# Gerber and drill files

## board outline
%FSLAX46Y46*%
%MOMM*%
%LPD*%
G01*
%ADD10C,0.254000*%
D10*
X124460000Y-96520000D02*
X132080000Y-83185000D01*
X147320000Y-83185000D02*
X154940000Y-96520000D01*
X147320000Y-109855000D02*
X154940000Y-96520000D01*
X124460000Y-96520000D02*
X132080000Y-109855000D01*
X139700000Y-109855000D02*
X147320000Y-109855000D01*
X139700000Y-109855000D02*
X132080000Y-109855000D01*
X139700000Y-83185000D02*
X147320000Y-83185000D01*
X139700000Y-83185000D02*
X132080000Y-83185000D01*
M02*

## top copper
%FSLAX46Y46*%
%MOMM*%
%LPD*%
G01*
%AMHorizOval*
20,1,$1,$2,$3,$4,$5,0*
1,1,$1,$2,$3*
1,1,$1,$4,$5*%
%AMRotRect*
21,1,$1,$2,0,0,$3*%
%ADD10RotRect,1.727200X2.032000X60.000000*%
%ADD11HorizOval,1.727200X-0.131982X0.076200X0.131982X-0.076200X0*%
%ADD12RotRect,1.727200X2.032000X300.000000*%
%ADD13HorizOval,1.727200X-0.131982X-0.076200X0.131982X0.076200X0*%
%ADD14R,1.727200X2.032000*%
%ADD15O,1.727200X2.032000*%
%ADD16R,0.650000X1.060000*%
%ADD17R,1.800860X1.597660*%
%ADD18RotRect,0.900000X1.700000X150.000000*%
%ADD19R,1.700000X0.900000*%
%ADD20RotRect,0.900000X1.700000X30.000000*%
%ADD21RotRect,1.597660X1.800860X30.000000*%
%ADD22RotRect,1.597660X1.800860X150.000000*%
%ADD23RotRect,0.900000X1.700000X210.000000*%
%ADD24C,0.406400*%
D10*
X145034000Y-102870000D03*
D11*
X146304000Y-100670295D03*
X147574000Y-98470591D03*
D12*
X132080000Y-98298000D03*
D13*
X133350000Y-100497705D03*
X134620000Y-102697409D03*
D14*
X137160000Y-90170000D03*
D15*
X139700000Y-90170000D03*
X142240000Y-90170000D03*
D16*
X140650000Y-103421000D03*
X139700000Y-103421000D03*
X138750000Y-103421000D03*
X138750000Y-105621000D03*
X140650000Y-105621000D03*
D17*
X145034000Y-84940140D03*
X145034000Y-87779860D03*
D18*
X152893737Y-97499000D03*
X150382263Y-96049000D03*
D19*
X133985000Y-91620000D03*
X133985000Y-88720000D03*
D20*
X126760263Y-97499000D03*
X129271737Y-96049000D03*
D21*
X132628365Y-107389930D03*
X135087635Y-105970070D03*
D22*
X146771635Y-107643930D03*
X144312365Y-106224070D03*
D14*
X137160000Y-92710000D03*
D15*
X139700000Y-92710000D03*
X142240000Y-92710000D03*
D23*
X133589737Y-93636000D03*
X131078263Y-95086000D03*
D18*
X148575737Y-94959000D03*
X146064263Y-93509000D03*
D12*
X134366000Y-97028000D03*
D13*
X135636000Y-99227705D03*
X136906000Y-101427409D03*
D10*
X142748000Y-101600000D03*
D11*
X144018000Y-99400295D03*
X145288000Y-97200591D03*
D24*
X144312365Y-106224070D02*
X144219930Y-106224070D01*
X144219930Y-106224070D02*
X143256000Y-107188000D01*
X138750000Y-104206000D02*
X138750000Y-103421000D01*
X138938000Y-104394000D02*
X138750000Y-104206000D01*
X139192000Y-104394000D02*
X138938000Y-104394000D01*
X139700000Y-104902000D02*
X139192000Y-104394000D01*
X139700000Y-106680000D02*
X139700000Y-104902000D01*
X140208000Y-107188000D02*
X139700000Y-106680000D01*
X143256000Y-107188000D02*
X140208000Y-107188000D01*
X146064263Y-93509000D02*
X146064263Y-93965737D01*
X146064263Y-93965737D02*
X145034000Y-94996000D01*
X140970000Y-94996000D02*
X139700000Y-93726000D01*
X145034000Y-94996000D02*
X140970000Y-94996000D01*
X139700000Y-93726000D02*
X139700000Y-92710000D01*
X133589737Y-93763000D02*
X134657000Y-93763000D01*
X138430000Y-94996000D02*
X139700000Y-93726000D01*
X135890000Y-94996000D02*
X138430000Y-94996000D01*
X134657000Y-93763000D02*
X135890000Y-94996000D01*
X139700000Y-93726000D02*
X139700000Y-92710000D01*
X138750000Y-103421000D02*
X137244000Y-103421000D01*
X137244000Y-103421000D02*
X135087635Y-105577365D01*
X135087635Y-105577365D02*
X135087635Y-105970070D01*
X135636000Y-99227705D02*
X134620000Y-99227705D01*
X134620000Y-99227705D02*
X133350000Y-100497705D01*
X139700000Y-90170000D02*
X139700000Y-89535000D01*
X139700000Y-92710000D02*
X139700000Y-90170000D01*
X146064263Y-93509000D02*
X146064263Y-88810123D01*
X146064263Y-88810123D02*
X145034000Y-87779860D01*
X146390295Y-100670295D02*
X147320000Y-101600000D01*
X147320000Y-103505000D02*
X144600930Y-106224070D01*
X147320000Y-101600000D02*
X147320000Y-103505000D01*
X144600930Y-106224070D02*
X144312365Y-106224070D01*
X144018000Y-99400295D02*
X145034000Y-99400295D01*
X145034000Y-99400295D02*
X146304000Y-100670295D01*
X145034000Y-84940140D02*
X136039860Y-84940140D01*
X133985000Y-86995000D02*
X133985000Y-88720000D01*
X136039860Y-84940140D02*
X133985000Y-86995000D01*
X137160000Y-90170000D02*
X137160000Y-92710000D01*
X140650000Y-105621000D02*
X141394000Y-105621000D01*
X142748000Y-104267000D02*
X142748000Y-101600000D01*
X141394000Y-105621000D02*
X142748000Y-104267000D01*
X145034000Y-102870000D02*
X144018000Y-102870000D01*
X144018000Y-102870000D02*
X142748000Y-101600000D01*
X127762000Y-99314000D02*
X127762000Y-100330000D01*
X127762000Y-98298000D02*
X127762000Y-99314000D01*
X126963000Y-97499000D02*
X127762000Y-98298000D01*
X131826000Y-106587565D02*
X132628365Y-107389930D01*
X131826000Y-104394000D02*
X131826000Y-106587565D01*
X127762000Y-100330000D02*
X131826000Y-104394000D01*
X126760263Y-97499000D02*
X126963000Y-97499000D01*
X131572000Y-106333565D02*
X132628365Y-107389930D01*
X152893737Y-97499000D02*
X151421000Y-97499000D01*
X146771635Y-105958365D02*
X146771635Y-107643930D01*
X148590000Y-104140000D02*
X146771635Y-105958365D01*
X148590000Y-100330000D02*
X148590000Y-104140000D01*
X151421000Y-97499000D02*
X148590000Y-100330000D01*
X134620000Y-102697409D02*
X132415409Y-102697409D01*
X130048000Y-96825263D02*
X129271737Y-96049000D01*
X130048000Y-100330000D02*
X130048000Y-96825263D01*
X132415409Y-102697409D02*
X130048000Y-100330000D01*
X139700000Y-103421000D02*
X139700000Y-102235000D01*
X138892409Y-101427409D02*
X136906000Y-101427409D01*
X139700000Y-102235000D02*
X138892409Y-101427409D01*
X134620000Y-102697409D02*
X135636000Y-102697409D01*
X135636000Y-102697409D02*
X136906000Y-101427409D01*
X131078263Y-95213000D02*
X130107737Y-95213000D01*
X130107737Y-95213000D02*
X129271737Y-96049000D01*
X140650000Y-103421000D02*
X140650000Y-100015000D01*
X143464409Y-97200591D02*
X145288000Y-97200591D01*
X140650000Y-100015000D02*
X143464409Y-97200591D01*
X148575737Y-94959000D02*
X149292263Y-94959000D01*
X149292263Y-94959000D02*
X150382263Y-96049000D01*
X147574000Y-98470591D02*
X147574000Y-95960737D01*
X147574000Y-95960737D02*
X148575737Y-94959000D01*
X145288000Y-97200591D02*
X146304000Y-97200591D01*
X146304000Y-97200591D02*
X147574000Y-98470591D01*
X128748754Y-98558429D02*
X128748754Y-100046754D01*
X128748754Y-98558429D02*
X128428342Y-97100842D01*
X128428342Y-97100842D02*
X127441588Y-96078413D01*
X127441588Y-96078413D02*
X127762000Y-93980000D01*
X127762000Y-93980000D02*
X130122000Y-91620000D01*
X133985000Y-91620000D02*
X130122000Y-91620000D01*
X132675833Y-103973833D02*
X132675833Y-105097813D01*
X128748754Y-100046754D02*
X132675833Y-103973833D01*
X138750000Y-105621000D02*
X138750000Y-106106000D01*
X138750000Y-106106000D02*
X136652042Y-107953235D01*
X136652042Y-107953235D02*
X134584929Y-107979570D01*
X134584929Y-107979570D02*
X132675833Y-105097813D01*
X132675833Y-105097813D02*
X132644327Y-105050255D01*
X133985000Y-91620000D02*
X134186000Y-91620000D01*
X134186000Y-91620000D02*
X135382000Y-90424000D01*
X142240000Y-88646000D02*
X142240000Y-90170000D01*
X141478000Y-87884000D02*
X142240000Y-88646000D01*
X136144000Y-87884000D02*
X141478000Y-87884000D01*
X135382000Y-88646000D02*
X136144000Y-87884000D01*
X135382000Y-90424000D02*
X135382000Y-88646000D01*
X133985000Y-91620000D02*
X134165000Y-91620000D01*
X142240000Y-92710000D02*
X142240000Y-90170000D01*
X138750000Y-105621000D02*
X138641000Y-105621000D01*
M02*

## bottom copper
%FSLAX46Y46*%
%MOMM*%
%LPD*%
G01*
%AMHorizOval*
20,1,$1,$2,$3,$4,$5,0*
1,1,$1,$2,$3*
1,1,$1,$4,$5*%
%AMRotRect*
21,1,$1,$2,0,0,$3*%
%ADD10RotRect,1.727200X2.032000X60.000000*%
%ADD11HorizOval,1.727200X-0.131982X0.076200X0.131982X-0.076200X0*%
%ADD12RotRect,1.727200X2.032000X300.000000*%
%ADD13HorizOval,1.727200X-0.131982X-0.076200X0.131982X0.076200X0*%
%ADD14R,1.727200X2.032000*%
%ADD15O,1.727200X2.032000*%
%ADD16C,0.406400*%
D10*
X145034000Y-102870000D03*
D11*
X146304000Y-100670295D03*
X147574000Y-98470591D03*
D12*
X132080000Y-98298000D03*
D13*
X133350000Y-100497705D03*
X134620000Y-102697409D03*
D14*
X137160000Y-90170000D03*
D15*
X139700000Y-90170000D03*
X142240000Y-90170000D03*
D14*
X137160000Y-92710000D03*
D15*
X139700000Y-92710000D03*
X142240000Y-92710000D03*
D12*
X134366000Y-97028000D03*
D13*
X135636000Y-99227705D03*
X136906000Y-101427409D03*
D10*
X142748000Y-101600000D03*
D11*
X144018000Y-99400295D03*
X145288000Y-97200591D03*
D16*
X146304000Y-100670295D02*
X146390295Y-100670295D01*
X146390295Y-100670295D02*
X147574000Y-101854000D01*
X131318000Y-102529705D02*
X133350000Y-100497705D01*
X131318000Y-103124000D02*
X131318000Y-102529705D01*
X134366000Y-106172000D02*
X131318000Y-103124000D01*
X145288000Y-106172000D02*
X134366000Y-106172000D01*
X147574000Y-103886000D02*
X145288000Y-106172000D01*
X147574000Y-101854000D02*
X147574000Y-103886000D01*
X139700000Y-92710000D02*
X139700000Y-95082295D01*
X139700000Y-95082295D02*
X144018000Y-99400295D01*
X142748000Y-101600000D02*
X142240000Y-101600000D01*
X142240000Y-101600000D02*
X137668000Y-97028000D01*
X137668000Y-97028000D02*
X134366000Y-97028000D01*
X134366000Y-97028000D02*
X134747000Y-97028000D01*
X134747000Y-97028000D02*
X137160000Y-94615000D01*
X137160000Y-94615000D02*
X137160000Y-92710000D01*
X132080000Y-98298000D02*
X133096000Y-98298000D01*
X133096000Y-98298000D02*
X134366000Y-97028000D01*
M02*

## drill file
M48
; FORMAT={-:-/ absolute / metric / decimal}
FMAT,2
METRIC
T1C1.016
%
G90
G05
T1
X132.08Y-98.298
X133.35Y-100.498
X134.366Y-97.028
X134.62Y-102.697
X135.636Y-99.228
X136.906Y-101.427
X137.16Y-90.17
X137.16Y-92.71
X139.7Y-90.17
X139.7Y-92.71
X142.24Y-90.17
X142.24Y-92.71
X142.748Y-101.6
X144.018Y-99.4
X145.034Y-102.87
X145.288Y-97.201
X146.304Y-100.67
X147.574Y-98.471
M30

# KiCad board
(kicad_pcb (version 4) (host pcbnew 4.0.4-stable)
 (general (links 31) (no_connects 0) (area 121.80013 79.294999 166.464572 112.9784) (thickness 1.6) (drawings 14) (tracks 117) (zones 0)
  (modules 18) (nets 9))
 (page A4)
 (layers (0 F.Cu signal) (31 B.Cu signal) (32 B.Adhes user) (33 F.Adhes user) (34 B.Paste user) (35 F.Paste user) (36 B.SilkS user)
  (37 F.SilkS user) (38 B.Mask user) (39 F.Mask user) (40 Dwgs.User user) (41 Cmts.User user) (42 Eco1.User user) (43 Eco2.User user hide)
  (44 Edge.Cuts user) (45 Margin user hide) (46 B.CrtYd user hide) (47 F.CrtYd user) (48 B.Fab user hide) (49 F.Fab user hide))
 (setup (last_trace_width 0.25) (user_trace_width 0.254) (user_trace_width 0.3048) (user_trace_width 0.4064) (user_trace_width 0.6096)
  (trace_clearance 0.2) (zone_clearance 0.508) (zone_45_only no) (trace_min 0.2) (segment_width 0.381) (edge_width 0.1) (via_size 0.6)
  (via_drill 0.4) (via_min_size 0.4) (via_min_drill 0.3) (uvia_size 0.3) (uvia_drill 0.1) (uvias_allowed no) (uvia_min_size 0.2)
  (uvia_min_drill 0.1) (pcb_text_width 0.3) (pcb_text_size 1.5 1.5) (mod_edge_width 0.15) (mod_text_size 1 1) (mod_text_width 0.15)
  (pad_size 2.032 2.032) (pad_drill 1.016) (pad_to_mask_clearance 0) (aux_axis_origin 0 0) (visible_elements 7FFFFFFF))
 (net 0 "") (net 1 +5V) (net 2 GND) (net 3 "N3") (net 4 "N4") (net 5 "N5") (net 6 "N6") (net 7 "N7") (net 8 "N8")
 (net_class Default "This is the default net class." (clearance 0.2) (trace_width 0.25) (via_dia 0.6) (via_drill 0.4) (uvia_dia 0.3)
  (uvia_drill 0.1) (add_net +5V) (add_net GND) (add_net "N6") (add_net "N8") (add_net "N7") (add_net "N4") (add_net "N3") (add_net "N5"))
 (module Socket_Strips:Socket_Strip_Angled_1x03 (layer F.Cu) (at 145.034 102.87 60)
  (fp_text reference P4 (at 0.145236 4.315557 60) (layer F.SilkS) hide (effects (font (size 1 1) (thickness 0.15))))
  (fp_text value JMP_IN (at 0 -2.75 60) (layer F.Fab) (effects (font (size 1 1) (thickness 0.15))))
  (pad 1 thru_hole rect (at 0 0 60) (size 1.7272 2.032) (drill 1.016) (layers *.Cu *.Mask F.SilkS) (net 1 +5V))
  (pad 2 thru_hole oval (at 2.54 0 60) (size 1.7272 2.032) (drill 1.016) (layers *.Cu *.Mask F.SilkS) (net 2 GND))
  (pad 3 thru_hole oval (at 5.08 0 60) (size 1.7272 2.032) (drill 1.016) (layers *.Cu *.Mask F.SilkS) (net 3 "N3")))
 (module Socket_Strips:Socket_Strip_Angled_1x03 (layer F.Cu) (at 132.08 98.298 300)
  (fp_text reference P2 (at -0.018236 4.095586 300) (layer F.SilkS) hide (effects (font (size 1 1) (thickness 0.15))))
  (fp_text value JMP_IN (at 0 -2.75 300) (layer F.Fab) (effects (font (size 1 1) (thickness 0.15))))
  (pad 1 thru_hole rect (at 0 0 300) (size 1.7272 2.032) (drill 1.016) (layers *.Cu *.Mask F.SilkS) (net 1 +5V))
  (pad 2 thru_hole oval (at 2.54 0 300) (size 1.7272 2.032) (drill 1.016) (layers *.Cu *.Mask F.SilkS) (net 2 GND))
  (pad 3 thru_hole oval (at 5.08 0 300) (size 1.7272 2.032) (drill 1.016) (layers *.Cu *.Mask F.SilkS) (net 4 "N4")))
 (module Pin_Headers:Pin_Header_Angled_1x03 (layer F.Cu) (at 137.16 90.17 90)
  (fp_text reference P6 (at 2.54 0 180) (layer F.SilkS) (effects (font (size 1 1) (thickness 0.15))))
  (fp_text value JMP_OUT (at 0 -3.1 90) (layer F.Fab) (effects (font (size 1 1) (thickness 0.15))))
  (pad 1 thru_hole rect (at 0 0 90) (size 2.032 1.7272) (drill 1.016) (layers *.Cu *.Mask F.SilkS) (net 1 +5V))
  (pad 2 thru_hole oval (at 0 2.54 90) (size 2.032 1.7272) (drill 1.016) (layers *.Cu *.Mask F.SilkS) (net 2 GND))
  (pad 3 thru_hole oval (at 0 5.08 90) (size 2.032 1.7272) (drill 1.016) (layers *.Cu *.Mask F.SilkS) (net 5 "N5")))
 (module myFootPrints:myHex (layer F.Cu) (at 139.7 96.52)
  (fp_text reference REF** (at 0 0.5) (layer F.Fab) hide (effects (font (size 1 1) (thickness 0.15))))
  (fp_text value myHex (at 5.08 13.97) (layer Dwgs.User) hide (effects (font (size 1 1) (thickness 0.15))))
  (fp_line (start -15.24 0) (end -7.62 -13.335) (layer Edge.Cuts) (width 0.254))
  (fp_line (start 7.62 -13.335) (end 15.24 0) (layer Edge.Cuts) (width 0.254))
  (fp_line (start 7.62 13.335) (end 15.24 0) (layer Edge.Cuts) (width 0.254))
  (fp_line (start -15.24 0) (end -7.62 13.335) (layer Edge.Cuts) (width 0.254))
  (fp_line (start 0 13.335) (end 7.62 13.335) (layer Edge.Cuts) (width 0.254))
  (fp_line (start 0 13.335) (end -7.62 13.335) (layer Edge.Cuts) (width 0.254))
  (fp_line (start 0 -13.335) (end 7.62 -13.335) (layer Edge.Cuts) (width 0.254))
  (fp_line (start 0 -13.335) (end -7.62 -13.335) (layer Edge.Cuts) (width 0.254)))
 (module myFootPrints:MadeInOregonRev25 (layer F.Cu) (at 131.699 92.837)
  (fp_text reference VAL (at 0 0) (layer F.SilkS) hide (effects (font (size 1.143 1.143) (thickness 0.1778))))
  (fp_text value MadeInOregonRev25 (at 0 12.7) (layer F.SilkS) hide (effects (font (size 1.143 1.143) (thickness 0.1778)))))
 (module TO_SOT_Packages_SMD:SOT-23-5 (layer F.Cu) (at 139.7 104.521 270)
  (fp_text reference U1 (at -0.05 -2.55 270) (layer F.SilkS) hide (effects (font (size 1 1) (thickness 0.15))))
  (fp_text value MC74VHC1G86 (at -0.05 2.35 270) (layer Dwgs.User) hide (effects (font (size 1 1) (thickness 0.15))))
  (pad 1 smd rect (at -1.1 -0.95 270) (size 1.06 0.65) (layers F.Cu F.Paste F.Mask) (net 3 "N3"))
  (pad 2 smd rect (at -1.1 0 270) (size 1.06 0.65) (layers F.Cu F.Paste F.Mask) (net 4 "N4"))
  (pad 3 smd rect (at -1.1 0.95 270) (size 1.06 0.65) (layers F.Cu F.Paste F.Mask) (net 2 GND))
  (pad 4 smd rect (at 1.1 0.95 270) (size 1.06 0.65) (layers F.Cu F.Paste F.Mask) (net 5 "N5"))
  (pad 5 smd rect (at 1.1 -0.95 270) (size 1.06 0.65) (layers F.Cu F.Paste F.Mask) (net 1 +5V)))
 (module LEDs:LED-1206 (layer F.Cu) (at 145.034 86.36 90)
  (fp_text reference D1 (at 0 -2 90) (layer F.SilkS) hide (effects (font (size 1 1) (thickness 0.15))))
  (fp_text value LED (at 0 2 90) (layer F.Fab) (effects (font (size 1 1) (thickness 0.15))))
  (pad 2 smd rect (at 1.41986 0 270) (size 1.59766 1.80086) (layers F.Cu F.Paste F.Mask) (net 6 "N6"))
  (pad 1 smd rect (at -1.41986 0 270) (size 1.59766 1.80086) (layers F.Cu F.Paste F.Mask) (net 2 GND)))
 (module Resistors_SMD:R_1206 (layer F.Cu) (at 151.638 96.774 150)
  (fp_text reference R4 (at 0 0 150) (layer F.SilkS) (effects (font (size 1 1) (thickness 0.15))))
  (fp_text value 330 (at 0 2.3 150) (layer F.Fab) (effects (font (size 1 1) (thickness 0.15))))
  (pad 1 smd rect (at -1.45 0 150) (size 0.9 1.7) (layers F.Cu F.Paste F.Mask) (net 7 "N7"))
  (pad 2 smd rect (at 1.45 0 150) (size 0.9 1.7) (layers F.Cu F.Paste F.Mask) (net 3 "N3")))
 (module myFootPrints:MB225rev (layer F.Cu) (at 147.447 92.71)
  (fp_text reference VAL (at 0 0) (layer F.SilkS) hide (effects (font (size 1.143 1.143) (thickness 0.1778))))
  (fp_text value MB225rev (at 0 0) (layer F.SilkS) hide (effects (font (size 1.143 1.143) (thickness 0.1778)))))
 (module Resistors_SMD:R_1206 (layer F.Cu) (at 133.985 90.17 90)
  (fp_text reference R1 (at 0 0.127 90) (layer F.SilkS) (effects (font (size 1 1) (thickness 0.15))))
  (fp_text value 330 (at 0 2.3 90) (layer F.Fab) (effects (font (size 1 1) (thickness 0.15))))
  (pad 1 smd rect (at -1.45 0 90) (size 0.9 1.7) (layers F.Cu F.Paste F.Mask) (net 5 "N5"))
  (pad 2 smd rect (at 1.45 0 90) (size 0.9 1.7) (layers F.Cu F.Paste F.Mask) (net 6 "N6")))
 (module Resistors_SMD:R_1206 (layer F.Cu) (at 128.016 96.774 30)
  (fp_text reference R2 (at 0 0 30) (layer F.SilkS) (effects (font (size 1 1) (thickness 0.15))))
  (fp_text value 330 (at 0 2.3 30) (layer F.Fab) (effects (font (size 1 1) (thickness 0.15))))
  (pad 1 smd rect (at -1.45 0 30) (size 0.9 1.7) (layers F.Cu F.Paste F.Mask) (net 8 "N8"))
  (pad 2 smd rect (at 1.45 0 30) (size 0.9 1.7) (layers F.Cu F.Paste F.Mask) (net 4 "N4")))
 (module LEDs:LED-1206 (layer F.Cu) (at 133.858 106.68 210)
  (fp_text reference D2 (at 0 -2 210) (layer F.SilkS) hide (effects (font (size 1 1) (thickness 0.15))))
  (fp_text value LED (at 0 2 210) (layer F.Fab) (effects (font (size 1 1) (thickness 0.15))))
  (pad 2 smd rect (at 1.41986 0 30) (size 1.59766 1.80086) (layers F.Cu F.Paste F.Mask) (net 8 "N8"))
  (pad 1 smd rect (at -1.41986 0 30) (size 1.59766 1.80086) (layers F.Cu F.Paste F.Mask) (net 2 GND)))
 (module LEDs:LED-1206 (layer F.Cu) (at 145.542 106.934 330)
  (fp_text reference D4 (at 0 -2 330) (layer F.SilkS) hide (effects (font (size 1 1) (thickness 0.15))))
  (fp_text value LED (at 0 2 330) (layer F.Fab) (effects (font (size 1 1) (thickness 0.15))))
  (pad 2 smd rect (at 1.41986 0 150) (size 1.59766 1.80086) (layers F.Cu F.Paste F.Mask) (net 7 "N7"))
  (pad 1 smd rect (at -1.41986 0 150) (size 1.59766 1.80086) (layers F.Cu F.Paste F.Mask) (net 2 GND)))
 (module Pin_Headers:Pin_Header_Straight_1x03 (layer F.Cu) (at 137.16 92.71 90)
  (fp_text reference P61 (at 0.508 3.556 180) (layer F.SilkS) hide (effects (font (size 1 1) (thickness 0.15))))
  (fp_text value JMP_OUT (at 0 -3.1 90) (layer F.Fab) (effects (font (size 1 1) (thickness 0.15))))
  (pad 1 thru_hole rect (at 0 0 90) (size 2.032 1.7272) (drill 1.016) (layers *.Cu *.Mask F.SilkS) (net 1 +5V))
  (pad 2 thru_hole oval (at 0 2.54 90) (size 2.032 1.7272) (drill 1.016) (layers *.Cu *.Mask F.SilkS) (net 2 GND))
  (pad 3 thru_hole oval (at 0 5.08 90) (size 2.032 1.7272) (drill 1.016) (layers *.Cu *.Mask F.SilkS) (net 5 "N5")))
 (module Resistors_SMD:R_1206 (layer F.Cu) (at 132.334 94.361 210)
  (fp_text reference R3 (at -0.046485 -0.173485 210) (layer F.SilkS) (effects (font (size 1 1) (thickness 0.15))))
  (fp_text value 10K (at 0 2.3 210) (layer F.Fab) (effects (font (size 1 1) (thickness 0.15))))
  (pad 1 smd rect (at -1.45 0 210) (size 0.9 1.7) (layers F.Cu F.Paste F.Mask) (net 2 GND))
  (pad 2 smd rect (at 1.45 0 210) (size 0.9 1.7) (layers F.Cu F.Paste F.Mask) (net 4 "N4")))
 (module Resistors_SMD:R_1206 (layer F.Cu) (at 147.32 94.234 150)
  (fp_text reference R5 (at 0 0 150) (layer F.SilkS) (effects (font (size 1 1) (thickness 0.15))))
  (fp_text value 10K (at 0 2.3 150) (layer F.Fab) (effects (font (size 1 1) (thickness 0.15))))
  (pad 1 smd rect (at -1.45 0 150) (size 0.9 1.7) (layers F.Cu F.Paste F.Mask) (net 3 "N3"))
  (pad 2 smd rect (at 1.45 0 150) (size 0.9 1.7) (layers F.Cu F.Paste F.Mask) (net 2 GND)))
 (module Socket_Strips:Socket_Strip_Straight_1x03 (layer F.Cu) (at 134.366 97.028 300)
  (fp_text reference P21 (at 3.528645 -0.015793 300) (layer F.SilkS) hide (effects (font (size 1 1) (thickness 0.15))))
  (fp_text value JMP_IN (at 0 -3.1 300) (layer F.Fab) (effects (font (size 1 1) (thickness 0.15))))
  (pad 1 thru_hole rect (at 0 0 300) (size 1.7272 2.032) (drill 1.016) (layers *.Cu *.Mask F.SilkS) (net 1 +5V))
  (pad 2 thru_hole oval (at 2.54 0 300) (size 1.7272 2.032) (drill 1.016) (layers *.Cu *.Mask F.SilkS) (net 2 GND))
  (pad 3 thru_hole oval (at 5.08 0 300) (size 1.7272 2.032) (drill 1.016) (layers *.Cu *.Mask F.SilkS) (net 4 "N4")))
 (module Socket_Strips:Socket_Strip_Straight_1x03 (layer F.Cu) (at 142.748 101.6 60)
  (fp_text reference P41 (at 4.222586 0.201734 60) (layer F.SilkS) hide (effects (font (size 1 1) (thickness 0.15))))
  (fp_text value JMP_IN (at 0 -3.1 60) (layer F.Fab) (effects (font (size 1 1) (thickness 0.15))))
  (pad 1 thru_hole rect (at 0 0 60) (size 1.7272 2.032) (drill 1.016) (layers *.Cu *.Mask F.SilkS) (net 1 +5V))
  (pad 2 thru_hole oval (at 2.54 0 60) (size 1.7272 2.032) (drill 1.016) (layers *.Cu *.Mask F.SilkS) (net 2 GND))
  (pad 3 thru_hole oval (at 5.08 0 60) (size 1.7272 2.032) (drill 1.016) (layers *.Cu *.Mask F.SilkS) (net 3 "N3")))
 (segment (start 144.312365 106.22407) (end 144.21993 106.22407) (width 0.4064) (layer F.Cu) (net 2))
 (segment (start 144.21993 106.22407) (end 143.256 107.188) (width 0.4064) (layer F.Cu) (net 2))
 (segment (start 138.75 104.206) (end 138.75 103.421) (width 0.4064) (layer F.Cu) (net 2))
 (segment (start 138.938 104.394) (end 138.75 104.206) (width 0.4064) (layer F.Cu) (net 2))
 (segment (start 139.192 104.394) (end 138.938 104.394) (width 0.4064) (layer F.Cu) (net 2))
 (segment (start 139.7 104.902) (end 139.192 104.394) (width 0.4064) (layer F.Cu) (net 2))
 (segment (start 139.7 106.68) (end 139.7 104.902) (width 0.4064) (layer F.Cu) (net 2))
 (segment (start 140.208 107.188) (end 139.7 106.68) (width 0.4064) (layer F.Cu) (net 2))
 (segment (start 143.256 107.188) (end 140.208 107.188) (width 0.4064) (layer F.Cu) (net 2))
 (segment (start 146.304 100.670295) (end 146.390295 100.670295) (width 0.4064) (layer B.Cu) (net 2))
 (segment (start 146.390295 100.670295) (end 147.574 101.854) (width 0.4064) (layer B.Cu) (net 2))
 (segment (start 131.318 102.529705) (end 133.35 100.497705) (width 0.4064) (layer B.Cu) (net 2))
 (segment (start 131.318 103.124) (end 131.318 102.529705) (width 0.4064) (layer B.Cu) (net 2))
 (segment (start 134.366 106.172) (end 131.318 103.124) (width 0.4064) (layer B.Cu) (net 2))
 (segment (start 145.288 106.172) (end 134.366 106.172) (width 0.4064) (layer B.Cu) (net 2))
 (segment (start 147.574 103.886) (end 145.288 106.172) (width 0.4064) (layer B.Cu) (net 2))
 (segment (start 147.574 101.854) (end 147.574 103.886) (width 0.4064) (layer B.Cu) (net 2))
 (segment (start 139.7 92.71) (end 139.7 95.082295) (width 0.4064) (layer B.Cu) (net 2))
 (segment (start 139.7 95.082295) (end 144.018 99.400295) (width 0.4064) (layer B.Cu) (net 2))
 (segment (start 146.064263 93.509) (end 146.064263 93.965737) (width 0.4064) (layer F.Cu) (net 2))
 (segment (start 146.064263 93.965737) (end 145.034 94.996) (width 0.4064) (layer F.Cu) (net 2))
 (segment (start 140.97 94.996) (end 139.7 93.726) (width 0.4064) (layer F.Cu) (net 2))
 (segment (start 145.034 94.996) (end 140.97 94.996) (width 0.4064) (layer F.Cu) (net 2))
 (segment (start 139.7 93.726) (end 139.7 92.71) (width 0.4064) (layer F.Cu) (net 2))
 (segment (start 133.589737 93.763) (end 134.657 93.763) (width 0.4064) (layer F.Cu) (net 2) (status 10))
 (segment (start 138.43 94.996) (end 139.7 93.726) (width 0.4064) (layer F.Cu) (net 2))
 (segment (start 135.89 94.996) (end 138.43 94.996) (width 0.4064) (layer F.Cu) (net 2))
 (segment (start 134.657 93.763) (end 135.89 94.996) (width 0.4064) (layer F.Cu) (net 2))
 (segment (start 139.7 93.726) (end 139.7 92.71) (width 0.4064) (layer F.Cu) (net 2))
 (segment (start 138.75 103.421) (end 137.244 103.421) (width 0.4064) (layer F.Cu) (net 2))
 (segment (start 137.244 103.421) (end 135.087635 105.577365) (width 0.4064) (layer F.Cu) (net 2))
 (segment (start 135.087635 105.577365) (end 135.087635 105.97007) (width 0.4064) (layer F.Cu) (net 2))
 (segment (start 135.636 99.227705) (end 134.62 99.227705) (width 0.4064) (layer F.Cu) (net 2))
 (segment (start 134.62 99.227705) (end 133.35 100.497705) (width 0.4064) (layer F.Cu) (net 2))
 (segment (start 139.7 90.17) (end 139.7 89.535) (width 0.4064) (layer F.Cu) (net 2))
 (segment (start 139.7 92.71) (end 139.7 90.17) (width 0.4064) (layer F.Cu) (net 2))
 (segment (start 146.064263 93.509) (end 146.064263 88.810123) (width 0.4064) (layer F.Cu) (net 2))
 (segment (start 146.064263 88.810123) (end 145.034 87.77986) (width 0.4064) (layer F.Cu) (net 2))
 (segment (start 146.390295 100.670295) (end 147.32 101.6) (width 0.4064) (layer F.Cu) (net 2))
 (segment (start 147.32 103.505) (end 144.60093 106.22407) (width 0.4064) (layer F.Cu) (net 2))
 (segment (start 147.32 101.6) (end 147.32 103.505) (width 0.4064) (layer F.Cu) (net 2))
 (segment (start 144.60093 106.22407) (end 144.312365 106.22407) (width 0.4064) (layer F.Cu) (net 2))
 (segment (start 144.018 99.400295) (end 145.034 99.400295) (width 0.4064) (layer F.Cu) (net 2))
 (segment (start 145.034 99.400295) (end 146.304 100.670295) (width 0.4064) (layer F.Cu) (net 2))
 (segment (start 145.034 84.94014) (end 136.03986 84.94014) (width 0.4064) (layer F.Cu) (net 6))
 (segment (start 133.985 86.995) (end 133.985 88.72) (width 0.4064) (layer F.Cu) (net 6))
 (segment (start 136.03986 84.94014) (end 133.985 86.995) (width 0.4064) (layer F.Cu) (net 6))
 (segment (start 142.748 101.6) (end 142.24 101.6) (width 0.4064) (layer B.Cu) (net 1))
 (segment (start 142.24 101.6) (end 137.668 97.028) (width 0.4064) (layer B.Cu) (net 1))
 (segment (start 137.668 97.028) (end 134.366 97.028) (width 0.4064) (layer B.Cu) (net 1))
 (segment (start 134.366 97.028) (end 134.747 97.028) (width 0.4064) (layer B.Cu) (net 1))
 (segment (start 134.747 97.028) (end 137.16 94.615) (width 0.4064) (layer B.Cu) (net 1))
 (segment (start 137.16 94.615) (end 137.16 92.71) (width 0.4064) (layer B.Cu) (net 1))
 (segment (start 132.08 98.298) (end 133.096 98.298) (width 0.4064) (layer B.Cu) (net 1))
 (segment (start 133.096 98.298) (end 134.366 97.028) (width 0.4064) (layer B.Cu) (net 1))
 (segment (start 137.16 90.17) (end 137.16 92.71) (width 0.4064) (layer F.Cu) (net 1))
 (segment (start 140.65 105.621) (end 141.394 105.621) (width 0.4064) (layer F.Cu) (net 1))
 (segment (start 142.748 104.267) (end 142.748 101.6) (width 0.4064) (layer F.Cu) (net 1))
 (segment (start 141.394 105.621) (end 142.748 104.267) (width 0.4064) (layer F.Cu) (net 1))
 (segment (start 145.034 102.87) (end 144.018 102.87) (width 0.4064) (layer F.Cu) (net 1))
 (segment (start 144.018 102.87) (end 142.748 101.6) (width 0.4064) (layer F.Cu) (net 1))
 (segment (start 127.762 99.314) (end 127.762 100.33) (width 0.4064) (layer F.Cu) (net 8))
 (segment (start 127.762 98.298) (end 127.762 99.314) (width 0.4064) (layer F.Cu) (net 8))
 (segment (start 126.963 97.499) (end 127.762 98.298) (width 0.4064) (layer F.Cu) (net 8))
 (segment (start 131.826 106.587565) (end 132.628365 107.38993) (width 0.4064) (layer F.Cu) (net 8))
 (segment (start 131.826 104.394) (end 131.826 106.587565) (width 0.4064) (layer F.Cu) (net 8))
 (segment (start 127.762 100.33) (end 131.826 104.394) (width 0.4064) (layer F.Cu) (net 8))
 (segment (start 126.760263 97.499) (end 126.963 97.499) (width 0.4064) (layer F.Cu) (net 8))
 (segment (start 131.572 106.333565) (end 132.628365 107.38993) (width 0.4064) (layer F.Cu) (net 8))
 (segment (start 152.893737 97.499) (end 151.421 97.499) (width 0.4064) (layer F.Cu) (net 7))
 (segment (start 146.771635 105.958365) (end 146.771635 107.64393) (width 0.4064) (layer F.Cu) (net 7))
 (segment (start 148.59 104.14) (end 146.771635 105.958365) (width 0.4064) (layer F.Cu) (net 7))
 (segment (start 148.59 100.33) (end 148.59 104.14) (width 0.4064) (layer F.Cu) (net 7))
 (segment (start 151.421 97.499) (end 148.59 100.33) (width 0.4064) (layer F.Cu) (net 7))
 (segment (start 134.62 102.697409) (end 132.415409 102.697409) (width 0.4064) (layer F.Cu) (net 4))
 (segment (start 130.048 96.825263) (end 129.271737 96.049) (width 0.4064) (layer F.Cu) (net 4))
 (segment (start 130.048 100.33) (end 130.048 96.825263) (width 0.4064) (layer F.Cu) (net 4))
 (segment (start 132.415409 102.697409) (end 130.048 100.33) (width 0.4064) (layer F.Cu) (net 4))
 (segment (start 139.7 103.421) (end 139.7 102.235) (width 0.4064) (layer F.Cu) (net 4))
 (segment (start 138.892409 101.427409) (end 136.906 101.427409) (width 0.4064) (layer F.Cu) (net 4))
 (segment (start 139.7 102.235) (end 138.892409 101.427409) (width 0.4064) (layer F.Cu) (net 4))
 (segment (start 134.62 102.697409) (end 135.636 102.697409) (width 0.4064) (layer F.Cu) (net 4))
 (segment (start 135.636 102.697409) (end 136.906 101.427409) (width 0.4064) (layer F.Cu) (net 4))
 (segment (start 131.078263 95.213) (end 130.107737 95.213) (width 0.4064) (layer F.Cu) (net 4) (status 10))
 (segment (start 130.107737 95.213) (end 129.271737 96.049) (width 0.4064) (layer F.Cu) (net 4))
 (segment (start 140.65 103.421) (end 140.65 100.015) (width 0.4064) (layer F.Cu) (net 3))
 (segment (start 143.464409 97.200591) (end 145.288 97.200591) (width 0.4064) (layer F.Cu) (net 3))
 (segment (start 140.65 100.015) (end 143.464409 97.200591) (width 0.4064) (layer F.Cu) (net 3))
 (segment (start 148.575737 94.959) (end 149.292263 94.959) (width 0.4064) (layer F.Cu) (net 3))
 (segment (start 149.292263 94.959) (end 150.382263 96.049) (width 0.4064) (layer F.Cu) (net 3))
 (segment (start 147.574 98.470591) (end 147.574 95.960737) (width 0.4064) (layer F.Cu) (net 3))
 (segment (start 147.574 95.960737) (end 148.575737 94.959) (width 0.4064) (layer F.Cu) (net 3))
 (segment (start 145.288 97.200591) (end 146.304 97.200591) (width 0.4064) (layer F.Cu) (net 3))
 (segment (start 146.304 97.200591) (end 147.574 98.470591) (width 0.4064) (layer F.Cu) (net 3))
 (segment (start 128.748754 98.558429) (end 128.748754 100.046754) (width 0.4064) (layer F.Cu) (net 5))
 (segment (start 128.748754 98.558429) (end 128.428342 97.100842) (width 0.4064) (layer F.Cu) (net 5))
 (segment (start 128.428342 97.100842) (end 127.441588 96.078413) (width 0.4064) (layer F.Cu) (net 5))
 (segment (start 127.441588 96.078413) (end 127.762 93.98) (width 0.4064) (layer F.Cu) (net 5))
 (segment (start 127.762 93.98) (end 130.122 91.62) (width 0.4064) (layer F.Cu) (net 5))
 (segment (start 133.985 91.62) (end 130.122 91.62) (width 0.4064) (layer F.Cu) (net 5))
 (segment (start 132.675833 103.973833) (end 132.675833 105.097813) (width 0.4064) (layer F.Cu) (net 5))
 (segment (start 128.748754 100.046754) (end 132.675833 103.973833) (width 0.4064) (layer F.Cu) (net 5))
 (segment (start 138.75 105.621) (end 138.75 106.106) (width 0.4064) (layer F.Cu) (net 5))
 (segment (start 138.75 106.106) (end 136.652042 107.953235) (width 0.4064) (layer F.Cu) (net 5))
 (segment (start 136.652042 107.953235) (end 134.584929 107.97957) (width 0.4064) (layer F.Cu) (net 5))
 (segment (start 134.584929 107.97957) (end 132.675833 105.097813) (width 0.4064) (layer F.Cu) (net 5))
 (segment (start 132.675833 105.097813) (end 132.644327 105.050255) (width 0.4064) (layer F.Cu) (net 5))
 (segment (start 133.985 91.62) (end 134.186 91.62) (width 0.4064) (layer F.Cu) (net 5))
 (segment (start 134.186 91.62) (end 135.382 90.424) (width 0.4064) (layer F.Cu) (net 5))
 (segment (start 142.24 88.646) (end 142.24 90.17) (width 0.4064) (layer F.Cu) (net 5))
 (segment (start 141.478 87.884) (end 142.24 88.646) (width 0.4064) (layer F.Cu) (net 5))
 (segment (start 136.144 87.884) (end 141.478 87.884) (width 0.4064) (layer F.Cu) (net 5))
 (segment (start 135.382 88.646) (end 136.144 87.884) (width 0.4064) (layer F.Cu) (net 5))
 (segment (start 135.382 90.424) (end 135.382 88.646) (width 0.4064) (layer F.Cu) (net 5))
 (segment (start 133.985 91.62) (end 134.165 91.62) (width 0.4064) (layer F.Cu) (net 5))
 (segment (start 142.24 92.71) (end 142.24 90.17) (width 0.4064) (layer F.Cu) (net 5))
 (segment (start 138.75 105.621) (end 138.641 105.621) (width 0.4064) (layer F.Cu) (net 5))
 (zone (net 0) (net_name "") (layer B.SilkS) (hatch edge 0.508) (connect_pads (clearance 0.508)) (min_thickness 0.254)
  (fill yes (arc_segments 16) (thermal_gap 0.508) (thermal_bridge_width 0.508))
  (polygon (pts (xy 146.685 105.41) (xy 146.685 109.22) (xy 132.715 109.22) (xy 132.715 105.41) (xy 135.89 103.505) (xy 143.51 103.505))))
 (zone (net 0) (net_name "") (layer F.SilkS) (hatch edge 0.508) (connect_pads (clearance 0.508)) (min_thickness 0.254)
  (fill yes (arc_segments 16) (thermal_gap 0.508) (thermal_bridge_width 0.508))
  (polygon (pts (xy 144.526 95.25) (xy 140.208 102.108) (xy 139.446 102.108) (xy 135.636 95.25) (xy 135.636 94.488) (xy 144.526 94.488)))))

